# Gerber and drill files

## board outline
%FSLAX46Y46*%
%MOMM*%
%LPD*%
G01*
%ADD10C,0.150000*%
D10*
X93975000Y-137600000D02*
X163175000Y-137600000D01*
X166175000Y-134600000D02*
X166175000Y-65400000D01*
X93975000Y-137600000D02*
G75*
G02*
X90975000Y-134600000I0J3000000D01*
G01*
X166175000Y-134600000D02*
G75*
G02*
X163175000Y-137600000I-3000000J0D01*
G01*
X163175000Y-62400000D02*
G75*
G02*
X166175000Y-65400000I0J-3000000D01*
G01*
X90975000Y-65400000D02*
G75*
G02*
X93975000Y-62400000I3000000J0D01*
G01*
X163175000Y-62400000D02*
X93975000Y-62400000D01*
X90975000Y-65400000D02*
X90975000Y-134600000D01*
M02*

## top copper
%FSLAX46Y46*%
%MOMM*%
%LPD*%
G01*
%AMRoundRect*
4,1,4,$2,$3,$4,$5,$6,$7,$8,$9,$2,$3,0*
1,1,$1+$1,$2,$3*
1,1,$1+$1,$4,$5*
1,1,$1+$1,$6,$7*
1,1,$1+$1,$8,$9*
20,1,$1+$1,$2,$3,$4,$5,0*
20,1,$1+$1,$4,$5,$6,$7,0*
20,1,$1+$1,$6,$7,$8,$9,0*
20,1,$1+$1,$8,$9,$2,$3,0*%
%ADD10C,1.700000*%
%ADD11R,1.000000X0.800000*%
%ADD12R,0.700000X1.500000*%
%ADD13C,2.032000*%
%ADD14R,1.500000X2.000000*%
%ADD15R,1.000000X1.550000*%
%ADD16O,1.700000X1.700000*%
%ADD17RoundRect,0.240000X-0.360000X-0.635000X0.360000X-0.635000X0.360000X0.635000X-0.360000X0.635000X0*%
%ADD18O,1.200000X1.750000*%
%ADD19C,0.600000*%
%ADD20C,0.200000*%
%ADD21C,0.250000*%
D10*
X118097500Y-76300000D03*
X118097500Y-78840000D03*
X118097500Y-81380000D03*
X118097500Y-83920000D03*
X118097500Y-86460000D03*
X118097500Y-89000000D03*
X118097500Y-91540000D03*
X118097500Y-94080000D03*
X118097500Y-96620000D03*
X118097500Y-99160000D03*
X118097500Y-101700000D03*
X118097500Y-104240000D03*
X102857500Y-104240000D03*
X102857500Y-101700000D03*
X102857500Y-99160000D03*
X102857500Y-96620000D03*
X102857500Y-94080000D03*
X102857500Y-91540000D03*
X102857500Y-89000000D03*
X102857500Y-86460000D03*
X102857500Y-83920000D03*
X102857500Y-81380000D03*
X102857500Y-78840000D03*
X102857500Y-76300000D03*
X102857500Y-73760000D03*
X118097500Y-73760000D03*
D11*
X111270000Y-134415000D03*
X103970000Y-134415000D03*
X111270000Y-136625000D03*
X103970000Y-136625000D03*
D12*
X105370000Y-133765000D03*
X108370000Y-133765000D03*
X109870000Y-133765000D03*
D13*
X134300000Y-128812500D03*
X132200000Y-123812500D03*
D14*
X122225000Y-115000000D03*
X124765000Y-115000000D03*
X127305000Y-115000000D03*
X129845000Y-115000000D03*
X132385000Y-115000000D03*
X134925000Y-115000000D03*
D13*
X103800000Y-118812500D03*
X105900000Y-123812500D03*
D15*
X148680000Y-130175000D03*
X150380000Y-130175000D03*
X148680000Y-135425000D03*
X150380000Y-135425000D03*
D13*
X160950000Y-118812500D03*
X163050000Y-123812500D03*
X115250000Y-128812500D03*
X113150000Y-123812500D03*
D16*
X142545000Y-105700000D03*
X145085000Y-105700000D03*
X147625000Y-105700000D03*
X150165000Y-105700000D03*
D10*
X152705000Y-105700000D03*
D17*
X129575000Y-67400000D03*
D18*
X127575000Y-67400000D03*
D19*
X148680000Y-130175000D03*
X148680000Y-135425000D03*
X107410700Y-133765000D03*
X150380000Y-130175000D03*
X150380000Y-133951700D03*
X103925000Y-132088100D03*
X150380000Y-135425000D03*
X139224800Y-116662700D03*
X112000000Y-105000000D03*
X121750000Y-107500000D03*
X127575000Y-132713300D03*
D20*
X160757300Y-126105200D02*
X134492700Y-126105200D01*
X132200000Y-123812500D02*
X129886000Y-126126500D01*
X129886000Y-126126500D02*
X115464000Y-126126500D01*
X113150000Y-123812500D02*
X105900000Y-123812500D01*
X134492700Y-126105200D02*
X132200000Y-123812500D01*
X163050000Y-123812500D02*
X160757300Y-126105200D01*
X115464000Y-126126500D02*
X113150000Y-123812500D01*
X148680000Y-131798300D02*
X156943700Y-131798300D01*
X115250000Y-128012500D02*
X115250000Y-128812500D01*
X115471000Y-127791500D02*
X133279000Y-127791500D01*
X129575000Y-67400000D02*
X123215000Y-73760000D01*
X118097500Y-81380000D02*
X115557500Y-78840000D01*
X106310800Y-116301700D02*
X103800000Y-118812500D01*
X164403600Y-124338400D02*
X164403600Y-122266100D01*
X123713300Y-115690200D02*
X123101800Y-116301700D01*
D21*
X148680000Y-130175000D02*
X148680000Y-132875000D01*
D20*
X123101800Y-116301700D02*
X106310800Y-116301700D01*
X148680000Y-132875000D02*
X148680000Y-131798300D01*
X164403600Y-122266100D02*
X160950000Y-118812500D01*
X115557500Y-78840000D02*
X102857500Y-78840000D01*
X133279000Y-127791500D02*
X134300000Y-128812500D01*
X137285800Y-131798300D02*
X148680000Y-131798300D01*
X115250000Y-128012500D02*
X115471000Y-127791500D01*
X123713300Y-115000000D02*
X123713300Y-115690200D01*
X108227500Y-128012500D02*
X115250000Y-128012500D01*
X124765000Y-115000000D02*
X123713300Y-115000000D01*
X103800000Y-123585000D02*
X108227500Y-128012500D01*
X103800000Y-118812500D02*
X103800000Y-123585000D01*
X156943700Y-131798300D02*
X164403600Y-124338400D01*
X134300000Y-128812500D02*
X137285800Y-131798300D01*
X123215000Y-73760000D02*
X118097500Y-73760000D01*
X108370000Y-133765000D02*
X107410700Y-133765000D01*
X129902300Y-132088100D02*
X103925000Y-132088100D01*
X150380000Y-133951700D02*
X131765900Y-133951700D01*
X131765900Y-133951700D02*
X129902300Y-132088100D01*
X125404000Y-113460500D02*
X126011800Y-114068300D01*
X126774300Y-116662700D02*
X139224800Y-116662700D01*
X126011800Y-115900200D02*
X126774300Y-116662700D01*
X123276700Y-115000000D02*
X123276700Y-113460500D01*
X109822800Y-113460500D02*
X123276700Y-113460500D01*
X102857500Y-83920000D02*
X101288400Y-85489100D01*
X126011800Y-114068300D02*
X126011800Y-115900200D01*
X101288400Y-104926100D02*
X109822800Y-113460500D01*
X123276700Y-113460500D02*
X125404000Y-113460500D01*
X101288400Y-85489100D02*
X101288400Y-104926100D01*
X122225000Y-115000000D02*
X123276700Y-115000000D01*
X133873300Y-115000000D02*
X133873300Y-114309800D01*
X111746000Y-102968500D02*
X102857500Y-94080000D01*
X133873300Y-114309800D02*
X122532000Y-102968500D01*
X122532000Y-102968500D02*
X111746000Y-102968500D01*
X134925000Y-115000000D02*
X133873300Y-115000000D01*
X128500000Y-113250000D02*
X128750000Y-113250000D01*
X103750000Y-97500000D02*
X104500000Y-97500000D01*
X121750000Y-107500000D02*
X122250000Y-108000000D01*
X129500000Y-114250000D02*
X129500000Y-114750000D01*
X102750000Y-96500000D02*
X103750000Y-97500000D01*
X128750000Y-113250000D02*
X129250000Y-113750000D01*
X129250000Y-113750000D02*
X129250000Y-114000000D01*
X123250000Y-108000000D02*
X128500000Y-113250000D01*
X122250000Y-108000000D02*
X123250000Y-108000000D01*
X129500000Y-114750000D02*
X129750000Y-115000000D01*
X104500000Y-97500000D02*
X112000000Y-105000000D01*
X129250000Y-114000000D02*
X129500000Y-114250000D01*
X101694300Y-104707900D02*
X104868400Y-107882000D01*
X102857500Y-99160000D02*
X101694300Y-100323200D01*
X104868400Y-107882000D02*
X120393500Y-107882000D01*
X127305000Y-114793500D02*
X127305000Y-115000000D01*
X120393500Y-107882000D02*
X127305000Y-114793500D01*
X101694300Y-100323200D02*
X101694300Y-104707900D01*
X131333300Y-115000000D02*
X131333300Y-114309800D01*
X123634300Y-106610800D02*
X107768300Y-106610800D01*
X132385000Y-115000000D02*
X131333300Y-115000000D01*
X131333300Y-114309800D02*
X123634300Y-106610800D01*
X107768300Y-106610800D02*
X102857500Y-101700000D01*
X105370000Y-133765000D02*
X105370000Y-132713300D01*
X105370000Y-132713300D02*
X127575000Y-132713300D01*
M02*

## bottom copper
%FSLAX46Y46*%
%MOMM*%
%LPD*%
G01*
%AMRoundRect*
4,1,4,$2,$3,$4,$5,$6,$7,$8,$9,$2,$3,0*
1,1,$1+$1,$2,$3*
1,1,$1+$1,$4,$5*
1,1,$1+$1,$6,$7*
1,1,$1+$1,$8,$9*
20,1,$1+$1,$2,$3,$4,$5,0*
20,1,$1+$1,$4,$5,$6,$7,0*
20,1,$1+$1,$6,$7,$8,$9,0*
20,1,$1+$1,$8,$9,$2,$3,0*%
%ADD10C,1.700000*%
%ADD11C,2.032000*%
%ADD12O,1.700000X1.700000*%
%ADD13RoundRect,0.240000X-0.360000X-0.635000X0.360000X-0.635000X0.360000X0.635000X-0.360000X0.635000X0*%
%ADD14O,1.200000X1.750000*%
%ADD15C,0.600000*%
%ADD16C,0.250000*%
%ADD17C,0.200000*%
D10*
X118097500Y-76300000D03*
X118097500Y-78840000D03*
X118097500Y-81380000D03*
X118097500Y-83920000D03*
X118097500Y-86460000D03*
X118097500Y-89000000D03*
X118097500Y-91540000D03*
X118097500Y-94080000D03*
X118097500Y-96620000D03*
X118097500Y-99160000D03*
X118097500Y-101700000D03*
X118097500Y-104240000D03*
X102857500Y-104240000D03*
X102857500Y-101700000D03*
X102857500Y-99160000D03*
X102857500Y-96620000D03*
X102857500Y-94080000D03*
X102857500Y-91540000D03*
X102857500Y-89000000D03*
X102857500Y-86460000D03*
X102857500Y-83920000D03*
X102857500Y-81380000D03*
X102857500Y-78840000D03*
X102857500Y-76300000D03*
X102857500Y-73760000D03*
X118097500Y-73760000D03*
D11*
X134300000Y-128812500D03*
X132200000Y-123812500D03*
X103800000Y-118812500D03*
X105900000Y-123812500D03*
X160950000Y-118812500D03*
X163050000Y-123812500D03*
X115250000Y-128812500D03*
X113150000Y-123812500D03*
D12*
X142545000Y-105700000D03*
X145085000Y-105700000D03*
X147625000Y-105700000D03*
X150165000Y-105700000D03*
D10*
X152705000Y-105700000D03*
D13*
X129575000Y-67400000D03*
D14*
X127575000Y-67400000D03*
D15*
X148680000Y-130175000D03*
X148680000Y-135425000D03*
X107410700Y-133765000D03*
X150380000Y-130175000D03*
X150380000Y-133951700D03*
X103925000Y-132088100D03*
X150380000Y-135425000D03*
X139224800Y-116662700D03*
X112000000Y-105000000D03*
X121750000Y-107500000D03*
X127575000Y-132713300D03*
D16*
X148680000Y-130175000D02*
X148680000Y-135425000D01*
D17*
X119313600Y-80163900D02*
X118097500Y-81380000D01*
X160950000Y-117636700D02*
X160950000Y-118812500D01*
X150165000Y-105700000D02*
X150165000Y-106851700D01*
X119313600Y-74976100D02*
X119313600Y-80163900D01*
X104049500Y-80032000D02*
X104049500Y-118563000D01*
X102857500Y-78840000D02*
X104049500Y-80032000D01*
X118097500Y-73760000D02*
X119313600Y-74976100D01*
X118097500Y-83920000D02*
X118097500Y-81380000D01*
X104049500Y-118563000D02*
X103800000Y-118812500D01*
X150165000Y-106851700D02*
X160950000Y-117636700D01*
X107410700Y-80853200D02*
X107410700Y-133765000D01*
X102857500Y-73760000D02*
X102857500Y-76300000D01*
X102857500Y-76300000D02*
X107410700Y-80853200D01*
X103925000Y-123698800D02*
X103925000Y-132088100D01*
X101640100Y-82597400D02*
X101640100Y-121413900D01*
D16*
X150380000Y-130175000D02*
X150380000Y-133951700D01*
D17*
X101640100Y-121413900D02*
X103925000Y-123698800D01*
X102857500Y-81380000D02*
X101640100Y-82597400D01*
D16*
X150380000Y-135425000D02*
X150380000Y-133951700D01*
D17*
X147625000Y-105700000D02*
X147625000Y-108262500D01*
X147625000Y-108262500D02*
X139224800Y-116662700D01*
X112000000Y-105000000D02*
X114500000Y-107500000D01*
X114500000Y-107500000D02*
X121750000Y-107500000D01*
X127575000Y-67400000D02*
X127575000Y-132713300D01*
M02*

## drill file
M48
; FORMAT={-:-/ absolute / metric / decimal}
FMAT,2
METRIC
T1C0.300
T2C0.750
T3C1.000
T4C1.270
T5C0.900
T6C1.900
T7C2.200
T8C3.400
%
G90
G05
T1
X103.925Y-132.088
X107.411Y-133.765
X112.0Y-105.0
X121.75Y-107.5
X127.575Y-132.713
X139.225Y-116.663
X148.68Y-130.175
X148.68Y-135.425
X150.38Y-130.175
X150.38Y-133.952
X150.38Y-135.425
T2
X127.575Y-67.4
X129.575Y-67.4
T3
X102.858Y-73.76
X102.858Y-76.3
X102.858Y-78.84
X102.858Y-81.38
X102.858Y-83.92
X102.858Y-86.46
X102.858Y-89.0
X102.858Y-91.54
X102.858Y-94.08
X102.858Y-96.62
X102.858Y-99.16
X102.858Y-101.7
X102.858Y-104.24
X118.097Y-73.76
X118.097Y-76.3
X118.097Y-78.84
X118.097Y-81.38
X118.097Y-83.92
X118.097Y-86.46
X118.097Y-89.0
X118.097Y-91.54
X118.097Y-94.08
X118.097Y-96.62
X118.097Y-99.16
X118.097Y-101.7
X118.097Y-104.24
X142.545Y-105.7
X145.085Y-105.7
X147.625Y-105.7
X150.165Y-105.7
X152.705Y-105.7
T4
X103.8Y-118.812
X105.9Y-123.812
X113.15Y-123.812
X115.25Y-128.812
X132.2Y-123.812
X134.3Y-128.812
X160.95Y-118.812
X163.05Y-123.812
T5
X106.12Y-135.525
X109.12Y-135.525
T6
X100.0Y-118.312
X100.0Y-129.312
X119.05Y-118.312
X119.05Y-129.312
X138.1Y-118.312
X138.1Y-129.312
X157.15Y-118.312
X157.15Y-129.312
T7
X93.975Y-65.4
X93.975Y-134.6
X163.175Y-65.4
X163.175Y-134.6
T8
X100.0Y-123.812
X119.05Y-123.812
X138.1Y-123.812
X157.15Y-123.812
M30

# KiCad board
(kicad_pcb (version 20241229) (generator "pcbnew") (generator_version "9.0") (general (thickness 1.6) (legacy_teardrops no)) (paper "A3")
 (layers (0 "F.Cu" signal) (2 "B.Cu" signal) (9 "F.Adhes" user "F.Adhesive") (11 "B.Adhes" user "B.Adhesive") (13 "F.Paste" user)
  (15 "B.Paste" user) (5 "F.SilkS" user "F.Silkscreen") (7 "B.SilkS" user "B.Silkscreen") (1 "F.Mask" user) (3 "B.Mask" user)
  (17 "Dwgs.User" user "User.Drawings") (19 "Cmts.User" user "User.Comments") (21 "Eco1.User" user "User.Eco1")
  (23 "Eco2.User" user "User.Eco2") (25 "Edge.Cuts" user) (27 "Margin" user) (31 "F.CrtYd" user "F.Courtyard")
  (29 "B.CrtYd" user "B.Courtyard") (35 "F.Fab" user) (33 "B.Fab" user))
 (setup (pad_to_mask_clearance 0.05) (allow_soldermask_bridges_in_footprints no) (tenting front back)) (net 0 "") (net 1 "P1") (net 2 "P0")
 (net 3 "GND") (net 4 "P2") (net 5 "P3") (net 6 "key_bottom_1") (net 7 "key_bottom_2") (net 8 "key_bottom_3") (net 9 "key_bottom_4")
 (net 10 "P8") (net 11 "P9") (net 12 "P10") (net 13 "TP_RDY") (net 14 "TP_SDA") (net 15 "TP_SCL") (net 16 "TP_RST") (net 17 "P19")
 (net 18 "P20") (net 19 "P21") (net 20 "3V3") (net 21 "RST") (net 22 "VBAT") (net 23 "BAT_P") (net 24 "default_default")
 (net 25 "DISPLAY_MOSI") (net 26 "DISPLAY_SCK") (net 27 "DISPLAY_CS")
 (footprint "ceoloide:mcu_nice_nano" (layer "F.Cu") (at 110.4775 89)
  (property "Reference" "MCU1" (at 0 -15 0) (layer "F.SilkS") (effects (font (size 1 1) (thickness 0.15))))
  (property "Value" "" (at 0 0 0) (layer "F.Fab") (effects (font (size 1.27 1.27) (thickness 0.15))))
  (pad "1" thru_hole circle (at 7.62 -12.7) (size 1.7 1.7) (drill 1) (layers "*.Cu" "*.Mask") (remove_unused_layers no) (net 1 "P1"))
  (pad "2" thru_hole circle (at 7.62 -10.16) (size 1.7 1.7) (drill 1) (layers "*.Cu" "*.Mask") (remove_unused_layers no) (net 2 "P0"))
  (pad "3" thru_hole circle (at 7.62 -7.62) (size 1.7 1.7) (drill 1) (layers "*.Cu" "*.Mask") (remove_unused_layers no) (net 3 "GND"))
  (pad "4" thru_hole circle (at 7.62 -5.08) (size 1.7 1.7) (drill 1) (layers "*.Cu" "*.Mask") (remove_unused_layers no) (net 3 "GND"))
  (pad "5" thru_hole circle (at 7.62 -2.54) (size 1.7 1.7) (drill 1) (layers "*.Cu" "*.Mask") (remove_unused_layers no) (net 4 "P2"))
  (pad "6" thru_hole circle (at 7.62 0) (size 1.7 1.7) (drill 1) (layers "*.Cu" "*.Mask") (remove_unused_layers no) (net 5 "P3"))
  (pad "7" thru_hole circle (at 7.62 2.54) (size 1.7 1.7) (drill 1) (layers "*.Cu" "*.Mask") (remove_unused_layers no)
   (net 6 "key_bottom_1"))
  (pad "8" thru_hole circle (at 7.62 5.08) (size 1.7 1.7) (drill 1) (layers "*.Cu" "*.Mask") (remove_unused_layers no)
   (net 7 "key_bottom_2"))
  (pad "9" thru_hole circle (at 7.62 7.62) (size 1.7 1.7) (drill 1) (layers "*.Cu" "*.Mask") (remove_unused_layers no)
   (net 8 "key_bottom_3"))
  (pad "10" thru_hole circle (at 7.62 10.16) (size 1.7 1.7) (drill 1) (layers "*.Cu" "*.Mask") (remove_unused_layers no)
   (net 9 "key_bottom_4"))
  (pad "11" thru_hole circle (at 7.62 12.7) (size 1.7 1.7) (drill 1) (layers "*.Cu" "*.Mask") (remove_unused_layers no) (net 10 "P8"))
  (pad "12" thru_hole circle (at 7.62 15.24) (size 1.7 1.7) (drill 1) (layers "*.Cu" "*.Mask") (remove_unused_layers no) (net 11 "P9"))
  (pad "13" thru_hole circle (at -7.62 15.24) (size 1.7 1.7) (drill 1) (layers "*.Cu" "*.Mask") (remove_unused_layers no) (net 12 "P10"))
  (pad "14" thru_hole circle (at -7.62 12.7) (size 1.7 1.7) (drill 1) (layers "*.Cu" "*.Mask") (remove_unused_layers no) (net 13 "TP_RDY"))
  (pad "15" thru_hole circle (at -7.62 10.16) (size 1.7 1.7) (drill 1) (layers "*.Cu" "*.Mask") (remove_unused_layers no) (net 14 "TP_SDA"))
  (pad "16" thru_hole circle (at -7.62 7.62) (size 1.7 1.7) (drill 1) (layers "*.Cu" "*.Mask") (remove_unused_layers no) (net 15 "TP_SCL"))
  (pad "17" thru_hole circle (at -7.62 5.08) (size 1.7 1.7) (drill 1) (layers "*.Cu" "*.Mask") (remove_unused_layers no) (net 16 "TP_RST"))
  (pad "18" thru_hole circle (at -7.62 2.54) (size 1.7 1.7) (drill 1) (layers "*.Cu" "*.Mask") (remove_unused_layers no) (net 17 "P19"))
  (pad "19" thru_hole circle (at -7.62 0) (size 1.7 1.7) (drill 1) (layers "*.Cu" "*.Mask") (remove_unused_layers no) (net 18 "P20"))
  (pad "20" thru_hole circle (at -7.62 -2.54) (size 1.7 1.7) (drill 1) (layers "*.Cu" "*.Mask") (remove_unused_layers no) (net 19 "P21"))
  (pad "21" thru_hole circle (at -7.62 -5.08) (size 1.7 1.7) (drill 1) (layers "*.Cu" "*.Mask") (remove_unused_layers no) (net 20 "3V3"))
  (pad "22" thru_hole circle (at -7.62 -7.62) (size 1.7 1.7) (drill 1) (layers "*.Cu" "*.Mask") (remove_unused_layers no) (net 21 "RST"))
  (pad "23" thru_hole circle (at -7.62 -10.16) (size 1.7 1.7) (drill 1) (layers "*.Cu" "*.Mask") (remove_unused_layers no) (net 3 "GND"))
  (pad "24" thru_hole circle (at -7.62 -12.7) (size 1.7 1.7) (drill 1) (layers "*.Cu" "*.Mask") (remove_unused_layers no) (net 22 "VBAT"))
  (pad "25" thru_hole circle (at -7.62 -15.24) (size 1.7 1.7) (drill 1) (layers "*.Cu" "*.Mask") (remove_unused_layers no) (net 22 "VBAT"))
  (pad "26" thru_hole circle (at 7.62 -15.24) (size 1.7 1.7) (drill 1) (layers "*.Cu" "*.Mask") (remove_unused_layers no) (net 3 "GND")))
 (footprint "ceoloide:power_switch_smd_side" (layer "F.Cu") (at 107.62 135.5 -90)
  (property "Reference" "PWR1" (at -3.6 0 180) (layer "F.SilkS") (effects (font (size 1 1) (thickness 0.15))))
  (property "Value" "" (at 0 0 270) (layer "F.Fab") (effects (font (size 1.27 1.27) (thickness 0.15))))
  (pad "" smd rect (at -1.085 -3.65) (size 1 0.8) (layers "F.Cu" "F.Mask" "F.Paste"))
  (pad "" smd rect (at -1.085 3.65) (size 1 0.8) (layers "F.Cu" "F.Mask" "F.Paste"))
  (pad "" np_thru_hole circle (at 0.025 -1.5) (size 0.9 0.9) (drill 0.9) (layers "*.Cu" "*.Mask"))
  (pad "" np_thru_hole circle (at 0.025 1.5) (size 0.9 0.9) (drill 0.9) (layers "*.Cu" "*.Mask"))
  (pad "" smd rect (at 1.125 -3.65) (size 1 0.8) (layers "F.Cu" "F.Mask" "F.Paste"))
  (pad "" smd rect (at 1.125 3.65) (size 1 0.8) (layers "F.Cu" "F.Mask" "F.Paste"))
  (pad "1" smd rect (at -1.735 2.25) (size 0.7 1.5) (layers "F.Cu" "F.Mask" "F.Paste") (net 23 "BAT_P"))
  (pad "2" smd rect (at -1.735 -0.75) (size 0.7 1.5) (layers "F.Cu" "F.Mask" "F.Paste") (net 22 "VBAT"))
  (pad "3" smd rect (at -1.735 -2.25) (size 0.7 1.5) (layers "F.Cu" "F.Mask" "F.Paste")))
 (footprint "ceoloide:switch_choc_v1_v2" (layer "F.Cu") (at 138.1 123.8125 90)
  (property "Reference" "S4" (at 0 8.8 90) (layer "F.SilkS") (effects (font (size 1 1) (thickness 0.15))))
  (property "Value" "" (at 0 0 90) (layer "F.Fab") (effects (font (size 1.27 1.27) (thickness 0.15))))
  (pad "" np_thru_hole circle (at -5.5 0 90) (size 1.9 1.9) (drill 1.9) (layers "*.Cu" "*.Mask"))
  (pad "" np_thru_hole circle (at 0 0 90) (size 3.4 3.4) (drill 3.4) (layers "*.Cu" "*.Mask"))
  (pad "" np_thru_hole circle (at 5.5 0 90) (size 1.9 1.9) (drill 1.9) (layers "*.Cu" "*.Mask"))
  (pad "1" thru_hole circle (at -5 -3.8 285) (size 2.032 2.032) (drill 1.27) (layers "*.Cu" "*.Mask") (remove_unused_layers no)
   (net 3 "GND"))
  (pad "2" thru_hole circle (at 0 -5.9 285) (size 2.032 2.032) (drill 1.27) (layers "*.Cu" "*.Mask") (remove_unused_layers no)
   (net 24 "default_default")))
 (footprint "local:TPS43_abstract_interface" (layer "F.Cu") (at 128.575 91)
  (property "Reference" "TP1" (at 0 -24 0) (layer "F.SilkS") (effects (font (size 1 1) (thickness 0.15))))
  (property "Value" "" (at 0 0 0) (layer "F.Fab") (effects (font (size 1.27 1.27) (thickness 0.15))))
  (pad "1" smd rect (at -6.35 24) (size 1.5 2) (layers "F.Cu" "F.Mask" "F.Paste") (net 20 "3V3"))
  (pad "2" smd rect (at -3.81 24) (size 1.5 2) (layers "F.Cu" "F.Mask" "F.Paste") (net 3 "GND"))
  (pad "3" smd rect (at -1.27 24) (size 1.5 2) (layers "F.Cu" "F.Mask" "F.Paste") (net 14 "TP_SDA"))
  (pad "4" smd rect (at 1.27 24) (size 1.5 2) (layers "F.Cu" "F.Mask" "F.Paste") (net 15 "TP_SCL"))
  (pad "5" smd rect (at 3.81 24) (size 1.5 2) (layers "F.Cu" "F.Mask" "F.Paste") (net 13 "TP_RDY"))
  (pad "6" smd rect (at 6.35 24) (size 1.5 2) (layers "F.Cu" "F.Mask" "F.Paste") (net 16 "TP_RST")))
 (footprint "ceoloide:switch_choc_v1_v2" (layer "F.Cu") (at 100 123.8125 -90)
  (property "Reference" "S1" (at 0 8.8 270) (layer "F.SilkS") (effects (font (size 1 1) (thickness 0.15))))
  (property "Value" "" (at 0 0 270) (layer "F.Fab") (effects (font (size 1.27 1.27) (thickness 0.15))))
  (pad "" np_thru_hole circle (at -5.5 0 270) (size 1.9 1.9) (drill 1.9) (layers "*.Cu" "*.Mask"))
  (pad "" np_thru_hole circle (at 0 0 270) (size 3.4 3.4) (drill 3.4) (layers "*.Cu" "*.Mask"))
  (pad "" np_thru_hole circle (at 5.5 0 270) (size 1.9 1.9) (drill 1.9) (layers "*.Cu" "*.Mask"))
  (pad "1" thru_hole circle (at -5 -3.8 105) (size 2.032 2.032) (drill 1.27) (layers "*.Cu" "*.Mask") (remove_unused_layers no)
   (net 3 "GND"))
  (pad "2" thru_hole circle (at 0 -5.9 105) (size 2.032 2.032) (drill 1.27) (layers "*.Cu" "*.Mask") (remove_unused_layers no)
   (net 24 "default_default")))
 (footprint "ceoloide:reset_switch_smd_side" (layer "F.Cu") (at 149.53 132.8 90)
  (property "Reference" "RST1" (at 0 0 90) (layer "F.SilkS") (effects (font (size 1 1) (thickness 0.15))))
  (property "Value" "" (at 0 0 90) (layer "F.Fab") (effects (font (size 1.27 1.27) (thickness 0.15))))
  (pad "1" smd rect (at 2.625 -0.85 270) (size 1.55 1) (layers "F.Cu" "F.Mask" "F.Paste") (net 3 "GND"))
  (pad "2" smd rect (at 2.625 0.85 270) (size 1.55 1) (layers "F.Cu" "F.Mask" "F.Paste") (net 21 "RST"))
  (pad "3" smd rect (at -2.625 -0.85 270) (size 1.55 1) (layers "F.Cu" "F.Mask" "F.Paste") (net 3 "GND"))
  (pad "4" smd rect (at -2.625 0.85 270) (size 1.55 1) (layers "F.Cu" "F.Mask" "F.Paste") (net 21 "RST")))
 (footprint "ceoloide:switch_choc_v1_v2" (layer "F.Cu") (at 157.15 123.8125 -90)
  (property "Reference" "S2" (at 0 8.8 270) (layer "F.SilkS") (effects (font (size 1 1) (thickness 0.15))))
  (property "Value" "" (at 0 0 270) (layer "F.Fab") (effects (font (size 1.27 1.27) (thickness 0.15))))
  (pad "" np_thru_hole circle (at -5.5 0 270) (size 1.9 1.9) (drill 1.9) (layers "*.Cu" "*.Mask"))
  (pad "" np_thru_hole circle (at 0 0 270) (size 3.4 3.4) (drill 3.4) (layers "*.Cu" "*.Mask"))
  (pad "" np_thru_hole circle (at 5.5 0 270) (size 1.9 1.9) (drill 1.9) (layers "*.Cu" "*.Mask"))
  (pad "1" thru_hole circle (at -5 -3.8 105) (size 2.032 2.032) (drill 1.27) (layers "*.Cu" "*.Mask") (remove_unused_layers no)
   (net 3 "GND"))
  (pad "2" thru_hole circle (at 0 -5.9 105) (size 2.032 2.032) (drill 1.27) (layers "*.Cu" "*.Mask") (remove_unused_layers no)
   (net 24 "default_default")))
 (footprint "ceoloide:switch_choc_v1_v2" (layer "F.Cu") (at 119.05 123.8125 90)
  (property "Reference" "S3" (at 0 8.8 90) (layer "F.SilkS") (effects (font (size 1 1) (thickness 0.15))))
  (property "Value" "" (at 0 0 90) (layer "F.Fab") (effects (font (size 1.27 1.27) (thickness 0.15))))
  (pad "" np_thru_hole circle (at -5.5 0 90) (size 1.9 1.9) (drill 1.9) (layers "*.Cu" "*.Mask"))
  (pad "" np_thru_hole circle (at 0 0 90) (size 3.4 3.4) (drill 3.4) (layers "*.Cu" "*.Mask"))
  (pad "" np_thru_hole circle (at 5.5 0 90) (size 1.9 1.9) (drill 1.9) (layers "*.Cu" "*.Mask"))
  (pad "1" thru_hole circle (at -5 -3.8 285) (size 2.032 2.032) (drill 1.27) (layers "*.Cu" "*.Mask") (remove_unused_layers no)
   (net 3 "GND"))
  (pad "2" thru_hole circle (at 0 -5.9 285) (size 2.032 2.032) (drill 1.27) (layers "*.Cu" "*.Mask") (remove_unused_layers no)
   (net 24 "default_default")))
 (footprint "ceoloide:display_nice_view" (layer "F.Cu") (at 147.625 89)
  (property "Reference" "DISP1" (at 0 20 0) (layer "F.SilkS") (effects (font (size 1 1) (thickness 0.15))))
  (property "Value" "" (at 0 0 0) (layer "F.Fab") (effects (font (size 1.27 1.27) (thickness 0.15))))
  (pad "1" thru_hole oval (at -5.08 16.7 270) (size 1.7 1.7) (drill 1) (layers "*.Cu" "*.Mask") (remove_unused_layers no)
   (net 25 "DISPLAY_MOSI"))
  (pad "2" thru_hole oval (at -2.54 16.7 270) (size 1.7 1.7) (drill 1) (layers "*.Cu" "*.Mask") (remove_unused_layers no)
   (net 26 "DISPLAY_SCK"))
  (pad "3" thru_hole oval (at 0 16.7 270) (size 1.7 1.7) (drill 1) (layers "*.Cu" "*.Mask") (remove_unused_layers no) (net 20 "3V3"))
  (pad "4" thru_hole oval (at 2.54 16.7 270) (size 1.7 1.7) (drill 1) (layers "*.Cu" "*.Mask") (remove_unused_layers no) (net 3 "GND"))
  (pad "5" thru_hole circle (at 5.08 16.7 270) (size 1.7 1.7) (drill 1) (layers "*.Cu" "*.Mask") (remove_unused_layers no)
   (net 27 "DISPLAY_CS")))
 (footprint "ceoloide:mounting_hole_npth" (layer "B.Cu") (at 93.975 134.6)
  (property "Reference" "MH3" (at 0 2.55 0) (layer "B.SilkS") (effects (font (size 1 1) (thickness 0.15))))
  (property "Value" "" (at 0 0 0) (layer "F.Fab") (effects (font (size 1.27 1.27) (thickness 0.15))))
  (pad "" np_thru_hole circle (at 0 0) (size 2.2 2.2) (drill 2.2) (layers "*.Cu" "*.Mask")))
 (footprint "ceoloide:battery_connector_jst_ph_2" (layer "B.Cu") (at 128.575 67.4)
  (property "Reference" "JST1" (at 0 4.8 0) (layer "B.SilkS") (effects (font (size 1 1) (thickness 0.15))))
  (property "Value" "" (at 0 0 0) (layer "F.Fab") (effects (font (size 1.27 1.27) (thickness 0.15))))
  (pad "1" thru_hole roundrect (at 1 0) (size 1.2 1.75) (drill 0.75) (layers "*.Cu" "*.Mask") (remove_unused_layers no)
   (roundrect_rratio 0.2) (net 3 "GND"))
  (pad "2" thru_hole oval (at -1 0) (size 1.2 1.75) (drill 0.75) (layers "*.Cu" "*.Mask") (remove_unused_layers no) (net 23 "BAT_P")))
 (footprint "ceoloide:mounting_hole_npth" (layer "B.Cu") (at 163.175 134.6)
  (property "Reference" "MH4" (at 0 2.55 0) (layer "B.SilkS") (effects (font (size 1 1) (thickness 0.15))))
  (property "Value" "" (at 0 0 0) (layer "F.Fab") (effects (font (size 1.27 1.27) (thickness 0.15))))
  (pad "" np_thru_hole circle (at 0 0) (size 2.2 2.2) (drill 2.2) (layers "*.Cu" "*.Mask")))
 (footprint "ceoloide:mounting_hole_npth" (layer "B.Cu") (at 163.175 65.4)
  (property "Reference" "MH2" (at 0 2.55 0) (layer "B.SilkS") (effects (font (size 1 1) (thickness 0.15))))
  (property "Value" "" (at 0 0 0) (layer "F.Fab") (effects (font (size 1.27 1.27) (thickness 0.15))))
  (pad "" np_thru_hole circle (at 0 0) (size 2.2 2.2) (drill 2.2) (layers "*.Cu" "*.Mask")))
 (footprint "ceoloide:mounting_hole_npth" (layer "B.Cu") (at 93.975 65.4)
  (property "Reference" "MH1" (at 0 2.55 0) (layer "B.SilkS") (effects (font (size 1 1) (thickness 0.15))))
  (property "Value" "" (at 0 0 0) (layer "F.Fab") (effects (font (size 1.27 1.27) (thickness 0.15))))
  (pad "" np_thru_hole circle (at 0 0) (size 2.2 2.2) (drill 2.2) (layers "*.Cu" "*.Mask")))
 (gr_line (start 93.975 137.6) (end 163.175 137.6) (stroke (width 0.15) (type default)) (layer "Edge.Cuts"))
 (gr_line (start 166.175 134.6) (end 166.175 65.4) (stroke (width 0.15) (type default)) (layer "Edge.Cuts"))
 (gr_arc (start 93.975 137.6) (mid 91.85368 136.72132) (end 90.975 134.6) (stroke (width 0.15) (type default)) (layer "Edge.Cuts"))
 (gr_arc (start 166.175 134.6) (mid 165.29632 136.72132) (end 163.175 137.6) (stroke (width 0.15) (type default)) (layer "Edge.Cuts"))
 (gr_arc (start 163.175 62.4) (mid 165.29632 63.27868) (end 166.175 65.4) (stroke (width 0.15) (type default)) (layer "Edge.Cuts"))
 (gr_arc (start 90.975 65.4) (mid 91.85368 63.27868) (end 93.975 62.4) (stroke (width 0.15) (type default)) (layer "Edge.Cuts"))
 (gr_line (start 163.175 62.4) (end 93.975 62.4) (stroke (width 0.15) (type default)) (layer "Edge.Cuts"))
 (gr_line (start 90.975 65.4) (end 90.975 134.6) (stroke (width 0.15) (type default)) (layer "Edge.Cuts"))
 (segment (start 160.7573 126.1052) (end 134.4927 126.1052) (width 0.2) (layer "F.Cu") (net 24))
 (segment (start 132.2 123.8125) (end 129.886 126.1265) (width 0.2) (layer "F.Cu") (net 24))
 (segment (start 129.886 126.1265) (end 115.464 126.1265) (width 0.2) (layer "F.Cu") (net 24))
 (segment (start 113.15 123.8125) (end 105.9 123.8125) (width 0.2) (layer "F.Cu") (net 24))
 (segment (start 134.4927 126.1052) (end 132.2 123.8125) (width 0.2) (layer "F.Cu") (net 24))
 (segment (start 163.05 123.8125) (end 160.7573 126.1052) (width 0.2) (layer "F.Cu") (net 24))
 (segment (start 115.464 126.1265) (end 113.15 123.8125) (width 0.2) (layer "F.Cu") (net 24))
 (segment (start 148.68 131.7983) (end 156.9437 131.7983) (width 0.2) (layer "F.Cu") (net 3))
 (segment (start 115.25 128.0125) (end 115.25 128.8125) (width 0.2) (layer "F.Cu") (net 3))
 (segment (start 115.471 127.7915) (end 133.279 127.7915) (width 0.2) (layer "F.Cu") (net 3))
 (segment (start 129.575 67.4) (end 123.215 73.76) (width 0.2) (layer "F.Cu") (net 3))
 (segment (start 118.0975 81.38) (end 115.5575 78.84) (width 0.2) (layer "F.Cu") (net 3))
 (segment (start 106.3108 116.3017) (end 103.8 118.8125) (width 0.2) (layer "F.Cu") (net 3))
 (segment (start 164.4036 124.3384) (end 164.4036 122.2661) (width 0.2) (layer "F.Cu") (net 3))
 (segment (start 123.7133 115.6902) (end 123.1018 116.3017) (width 0.2) (layer "F.Cu") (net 3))
 (segment (start 148.68 130.175) (end 148.68 132.875) (width 0.25) (layer "F.Cu") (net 3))
 (segment (start 123.1018 116.3017) (end 106.3108 116.3017) (width 0.2) (layer "F.Cu") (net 3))
 (segment (start 148.68 132.875) (end 148.68 131.7983) (width 0.2) (layer "F.Cu") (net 3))
 (segment (start 164.4036 122.2661) (end 160.95 118.8125) (width 0.2) (layer "F.Cu") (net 3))
 (segment (start 115.5575 78.84) (end 102.8575 78.84) (width 0.2) (layer "F.Cu") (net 3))
 (segment (start 133.279 127.7915) (end 134.3 128.8125) (width 0.2) (layer "F.Cu") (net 3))
 (segment (start 137.2858 131.7983) (end 148.68 131.7983) (width 0.2) (layer "F.Cu") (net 3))
 (segment (start 115.25 128.0125) (end 115.471 127.7915) (width 0.2) (layer "F.Cu") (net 3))
 (segment (start 123.7133 115) (end 123.7133 115.6902) (width 0.2) (layer "F.Cu") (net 3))
 (segment (start 108.2275 128.0125) (end 115.25 128.0125) (width 0.2) (layer "F.Cu") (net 3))
 (segment (start 124.765 115) (end 123.7133 115) (width 0.2) (layer "F.Cu") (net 3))
 (segment (start 103.8 123.585) (end 108.2275 128.0125) (width 0.2) (layer "F.Cu") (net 3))
 (segment (start 103.8 118.8125) (end 103.8 123.585) (width 0.2) (layer "F.Cu") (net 3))
 (segment (start 156.9437 131.7983) (end 164.4036 124.3384) (width 0.2) (layer "F.Cu") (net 3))
 (segment (start 134.3 128.8125) (end 137.2858 131.7983) (width 0.2) (layer "F.Cu") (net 3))
 (segment (start 123.215 73.76) (end 118.0975 73.76) (width 0.2) (layer "F.Cu") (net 3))
 (via (at 148.68 130.175) (size 0.6) (drill 0.3) (layers "F.Cu" "B.Cu") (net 3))
 (via (at 148.68 135.425) (size 0.6) (drill 0.3) (layers "F.Cu" "B.Cu") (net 3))
 (segment (start 148.68 130.175) (end 148.68 135.425) (width 0.25) (layer "B.Cu") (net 3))
 (segment (start 119.3136 80.1639) (end 118.0975 81.38) (width 0.2) (layer "B.Cu") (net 3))
 (segment (start 160.95 117.6367) (end 160.95 118.8125) (width 0.2) (layer "B.Cu") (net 3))
 (segment (start 150.165 105.7) (end 150.165 106.8517) (width 0.2) (layer "B.Cu") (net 3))
 (segment (start 119.3136 74.9761) (end 119.3136 80.1639) (width 0.2) (layer "B.Cu") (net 3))
 (segment (start 104.0495 80.032) (end 104.0495 118.563) (width 0.2) (layer "B.Cu") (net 3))
 (segment (start 102.8575 78.84) (end 104.0495 80.032) (width 0.2) (layer "B.Cu") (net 3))
 (segment (start 118.0975 73.76) (end 119.3136 74.9761) (width 0.2) (layer "B.Cu") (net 3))
 (segment (start 118.0975 83.92) (end 118.0975 81.38) (width 0.2) (layer "B.Cu") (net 3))
 (segment (start 104.0495 118.563) (end 103.8 118.8125) (width 0.2) (layer "B.Cu") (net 3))
 (segment (start 150.165 106.8517) (end 160.95 117.6367) (width 0.2) (layer "B.Cu") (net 3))
 (segment (start 108.37 133.765) (end 107.4107 133.765) (width 0.2) (layer "F.Cu") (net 22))
 (via (at 107.4107 133.765) (size 0.6) (drill 0.3) (layers "F.Cu" "B.Cu") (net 22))
 (segment (start 107.4107 80.8532) (end 107.4107 133.765) (width 0.2) (layer "B.Cu") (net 22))
 (segment (start 102.8575 73.76) (end 102.8575 76.3) (width 0.2) (layer "B.Cu") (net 22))
 (segment (start 102.8575 76.3) (end 107.4107 80.8532) (width 0.2) (layer "B.Cu") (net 22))
 (segment (start 129.9023 132.0881) (end 103.925 132.0881) (width 0.2) (layer "F.Cu") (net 21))
 (segment (start 150.38 133.9517) (end 131.7659 133.9517) (width 0.2) (layer "F.Cu") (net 21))
 (segment (start 131.7659 133.9517) (end 129.9023 132.0881) (width 0.2) (layer "F.Cu") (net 21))
 (via (at 150.38 130.175) (size 0.6) (drill 0.3) (layers "F.Cu" "B.Cu") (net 21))
 (via (at 150.38 133.9517) (size 0.6) (drill 0.3) (layers "F.Cu" "B.Cu") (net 21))
 (via (at 103.925 132.0881) (size 0.6) (drill 0.3) (layers "F.Cu" "B.Cu") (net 21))
 (via (at 150.38 135.425) (size 0.6) (drill 0.3) (layers "F.Cu" "B.Cu") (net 21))
 (segment (start 103.925 123.6988) (end 103.925 132.0881) (width 0.2) (layer "B.Cu") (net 21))
 (segment (start 101.6401 82.5974) (end 101.6401 121.4139) (width 0.2) (layer "B.Cu") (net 21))
 (segment (start 150.38 130.175) (end 150.38 133.9517) (width 0.25) (layer "B.Cu") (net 21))
 (segment (start 101.6401 121.4139) (end 103.925 123.6988) (width 0.2) (layer "B.Cu") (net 21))
 (segment (start 102.8575 81.38) (end 101.6401 82.5974) (width 0.2) (layer "B.Cu") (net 21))
 (segment (start 150.38 135.425) (end 150.38 133.9517) (width 0.25) (layer "B.Cu") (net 21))
 (segment (start 125.404 113.4605) (end 126.0118 114.0683) (width 0.2) (layer "F.Cu") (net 20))
 (segment (start 126.7743 116.6627) (end 139.2248 116.6627) (width 0.2) (layer "F.Cu") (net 20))
 (segment (start 126.0118 115.9002) (end 126.7743 116.6627) (width 0.2) (layer "F.Cu") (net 20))
 (segment (start 123.2767 115) (end 123.2767 113.4605) (width 0.2) (layer "F.Cu") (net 20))
 (segment (start 109.8228 113.4605) (end 123.2767 113.4605) (width 0.2) (layer "F.Cu") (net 20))
 (segment (start 102.8575 83.92) (end 101.2884 85.4891) (width 0.2) (layer "F.Cu") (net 20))
 (segment (start 126.0118 114.0683) (end 126.0118 115.9002) (width 0.2) (layer "F.Cu") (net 20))
 (segment (start 101.2884 104.9261) (end 109.8228 113.4605) (width 0.2) (layer "F.Cu") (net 20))
 (segment (start 123.2767 113.4605) (end 125.404 113.4605) (width 0.2) (layer "F.Cu") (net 20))
 (segment (start 101.2884 85.4891) (end 101.2884 104.9261) (width 0.2) (layer "F.Cu") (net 20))
 (segment (start 122.225 115) (end 123.2767 115) (width 0.2) (layer "F.Cu") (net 20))
 (via (at 139.2248 116.6627) (size 0.6) (drill 0.3) (layers "F.Cu" "B.Cu") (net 20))
 (segment (start 147.625 105.7) (end 147.625 108.2625) (width 0.2) (layer "B.Cu") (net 20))
 (segment (start 147.625 108.2625) (end 139.2248 116.6627) (width 0.2) (layer "B.Cu") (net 20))
 (segment (start 133.8733 115) (end 133.8733 114.3098) (width 0.2) (layer "F.Cu") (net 16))
 (segment (start 111.746 102.9685) (end 102.8575 94.08) (width 0.2) (layer "F.Cu") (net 16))
 (segment (start 133.8733 114.3098) (end 122.532 102.9685) (width 0.2) (layer "F.Cu") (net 16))
 (segment (start 122.532 102.9685) (end 111.746 102.9685) (width 0.2) (layer "F.Cu") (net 16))
 (segment (start 134.925 115) (end 133.8733 115) (width 0.2) (layer "F.Cu") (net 16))
 (segment (start 128.5 113.25) (end 128.75 113.25) (width 0.2) (layer "F.Cu") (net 15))
 (segment (start 103.75 97.5) (end 104.5 97.5) (width 0.2) (layer "F.Cu") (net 15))
 (segment (start 121.75 107.5) (end 122.25 108) (width 0.2) (layer "F.Cu") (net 15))
 (segment (start 129.5 114.25) (end 129.5 114.75) (width 0.2) (layer "F.Cu") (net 15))
 (segment (start 102.75 96.5) (end 103.75 97.5) (width 0.2) (layer "F.Cu") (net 15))
 (segment (start 128.75 113.25) (end 129.25 113.75) (width 0.2) (layer "F.Cu") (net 15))
 (segment (start 129.25 113.75) (end 129.25 114) (width 0.2) (layer "F.Cu") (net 15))
 (segment (start 123.25 108) (end 128.5 113.25) (width 0.2) (layer "F.Cu") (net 15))
 (segment (start 122.25 108) (end 123.25 108) (width 0.2) (layer "F.Cu") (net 15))
 (segment (start 129.5 114.75) (end 129.75 115) (width 0.2) (layer "F.Cu") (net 15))
 (segment (start 104.5 97.5) (end 112 105) (width 0.2) (layer "F.Cu") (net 15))
 (segment (start 129.25 114) (end 129.5 114.25) (width 0.2) (layer "F.Cu") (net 15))
 (via (at 112 105) (size 0.6) (drill 0.3) (layers "F.Cu" "B.Cu") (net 15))
 (via (at 121.75 107.5) (size 0.6) (drill 0.3) (layers "F.Cu" "B.Cu") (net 15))
 (segment (start 112 105) (end 114.5 107.5) (width 0.2) (layer "B.Cu") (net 15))
 (segment (start 114.5 107.5) (end 121.75 107.5) (width 0.2) (layer "B.Cu") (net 15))
 (segment (start 101.6943 104.7079) (end 104.8684 107.882) (width 0.2) (layer "F.Cu") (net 14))
 (segment (start 102.8575 99.16) (end 101.6943 100.3232) (width 0.2) (layer "F.Cu") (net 14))
 (segment (start 104.8684 107.882) (end 120.3935 107.882) (width 0.2) (layer "F.Cu") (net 14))
 (segment (start 127.305 114.7935) (end 127.305 115) (width 0.2) (layer "F.Cu") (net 14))
 (segment (start 120.3935 107.882) (end 127.305 114.7935) (width 0.2) (layer "F.Cu") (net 14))
 (segment (start 101.6943 100.3232) (end 101.6943 104.7079) (width 0.2) (layer "F.Cu") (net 14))
 (segment (start 131.3333 115) (end 131.3333 114.3098) (width 0.2) (layer "F.Cu") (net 13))
 (segment (start 123.6343 106.6108) (end 107.7683 106.6108) (width 0.2) (layer "F.Cu") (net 13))
 (segment (start 132.385 115) (end 131.3333 115) (width 0.2) (layer "F.Cu") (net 13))
 (segment (start 131.3333 114.3098) (end 123.6343 106.6108) (width 0.2) (layer "F.Cu") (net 13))
 (segment (start 107.7683 106.6108) (end 102.8575 101.7) (width 0.2) (layer "F.Cu") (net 13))
 (segment (start 105.37 133.765) (end 105.37 132.7133) (width 0.2) (layer "F.Cu") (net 23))
 (segment (start 105.37 132.7133) (end 127.575 132.7133) (width 0.2) (layer "F.Cu") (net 23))
 (via (at 127.575 132.7133) (size 0.6) (drill 0.3) (layers "F.Cu" "B.Cu") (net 23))
 (segment (start 127.575 67.4) (end 127.575 132.7133) (width 0.2) (layer "B.Cu") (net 23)))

